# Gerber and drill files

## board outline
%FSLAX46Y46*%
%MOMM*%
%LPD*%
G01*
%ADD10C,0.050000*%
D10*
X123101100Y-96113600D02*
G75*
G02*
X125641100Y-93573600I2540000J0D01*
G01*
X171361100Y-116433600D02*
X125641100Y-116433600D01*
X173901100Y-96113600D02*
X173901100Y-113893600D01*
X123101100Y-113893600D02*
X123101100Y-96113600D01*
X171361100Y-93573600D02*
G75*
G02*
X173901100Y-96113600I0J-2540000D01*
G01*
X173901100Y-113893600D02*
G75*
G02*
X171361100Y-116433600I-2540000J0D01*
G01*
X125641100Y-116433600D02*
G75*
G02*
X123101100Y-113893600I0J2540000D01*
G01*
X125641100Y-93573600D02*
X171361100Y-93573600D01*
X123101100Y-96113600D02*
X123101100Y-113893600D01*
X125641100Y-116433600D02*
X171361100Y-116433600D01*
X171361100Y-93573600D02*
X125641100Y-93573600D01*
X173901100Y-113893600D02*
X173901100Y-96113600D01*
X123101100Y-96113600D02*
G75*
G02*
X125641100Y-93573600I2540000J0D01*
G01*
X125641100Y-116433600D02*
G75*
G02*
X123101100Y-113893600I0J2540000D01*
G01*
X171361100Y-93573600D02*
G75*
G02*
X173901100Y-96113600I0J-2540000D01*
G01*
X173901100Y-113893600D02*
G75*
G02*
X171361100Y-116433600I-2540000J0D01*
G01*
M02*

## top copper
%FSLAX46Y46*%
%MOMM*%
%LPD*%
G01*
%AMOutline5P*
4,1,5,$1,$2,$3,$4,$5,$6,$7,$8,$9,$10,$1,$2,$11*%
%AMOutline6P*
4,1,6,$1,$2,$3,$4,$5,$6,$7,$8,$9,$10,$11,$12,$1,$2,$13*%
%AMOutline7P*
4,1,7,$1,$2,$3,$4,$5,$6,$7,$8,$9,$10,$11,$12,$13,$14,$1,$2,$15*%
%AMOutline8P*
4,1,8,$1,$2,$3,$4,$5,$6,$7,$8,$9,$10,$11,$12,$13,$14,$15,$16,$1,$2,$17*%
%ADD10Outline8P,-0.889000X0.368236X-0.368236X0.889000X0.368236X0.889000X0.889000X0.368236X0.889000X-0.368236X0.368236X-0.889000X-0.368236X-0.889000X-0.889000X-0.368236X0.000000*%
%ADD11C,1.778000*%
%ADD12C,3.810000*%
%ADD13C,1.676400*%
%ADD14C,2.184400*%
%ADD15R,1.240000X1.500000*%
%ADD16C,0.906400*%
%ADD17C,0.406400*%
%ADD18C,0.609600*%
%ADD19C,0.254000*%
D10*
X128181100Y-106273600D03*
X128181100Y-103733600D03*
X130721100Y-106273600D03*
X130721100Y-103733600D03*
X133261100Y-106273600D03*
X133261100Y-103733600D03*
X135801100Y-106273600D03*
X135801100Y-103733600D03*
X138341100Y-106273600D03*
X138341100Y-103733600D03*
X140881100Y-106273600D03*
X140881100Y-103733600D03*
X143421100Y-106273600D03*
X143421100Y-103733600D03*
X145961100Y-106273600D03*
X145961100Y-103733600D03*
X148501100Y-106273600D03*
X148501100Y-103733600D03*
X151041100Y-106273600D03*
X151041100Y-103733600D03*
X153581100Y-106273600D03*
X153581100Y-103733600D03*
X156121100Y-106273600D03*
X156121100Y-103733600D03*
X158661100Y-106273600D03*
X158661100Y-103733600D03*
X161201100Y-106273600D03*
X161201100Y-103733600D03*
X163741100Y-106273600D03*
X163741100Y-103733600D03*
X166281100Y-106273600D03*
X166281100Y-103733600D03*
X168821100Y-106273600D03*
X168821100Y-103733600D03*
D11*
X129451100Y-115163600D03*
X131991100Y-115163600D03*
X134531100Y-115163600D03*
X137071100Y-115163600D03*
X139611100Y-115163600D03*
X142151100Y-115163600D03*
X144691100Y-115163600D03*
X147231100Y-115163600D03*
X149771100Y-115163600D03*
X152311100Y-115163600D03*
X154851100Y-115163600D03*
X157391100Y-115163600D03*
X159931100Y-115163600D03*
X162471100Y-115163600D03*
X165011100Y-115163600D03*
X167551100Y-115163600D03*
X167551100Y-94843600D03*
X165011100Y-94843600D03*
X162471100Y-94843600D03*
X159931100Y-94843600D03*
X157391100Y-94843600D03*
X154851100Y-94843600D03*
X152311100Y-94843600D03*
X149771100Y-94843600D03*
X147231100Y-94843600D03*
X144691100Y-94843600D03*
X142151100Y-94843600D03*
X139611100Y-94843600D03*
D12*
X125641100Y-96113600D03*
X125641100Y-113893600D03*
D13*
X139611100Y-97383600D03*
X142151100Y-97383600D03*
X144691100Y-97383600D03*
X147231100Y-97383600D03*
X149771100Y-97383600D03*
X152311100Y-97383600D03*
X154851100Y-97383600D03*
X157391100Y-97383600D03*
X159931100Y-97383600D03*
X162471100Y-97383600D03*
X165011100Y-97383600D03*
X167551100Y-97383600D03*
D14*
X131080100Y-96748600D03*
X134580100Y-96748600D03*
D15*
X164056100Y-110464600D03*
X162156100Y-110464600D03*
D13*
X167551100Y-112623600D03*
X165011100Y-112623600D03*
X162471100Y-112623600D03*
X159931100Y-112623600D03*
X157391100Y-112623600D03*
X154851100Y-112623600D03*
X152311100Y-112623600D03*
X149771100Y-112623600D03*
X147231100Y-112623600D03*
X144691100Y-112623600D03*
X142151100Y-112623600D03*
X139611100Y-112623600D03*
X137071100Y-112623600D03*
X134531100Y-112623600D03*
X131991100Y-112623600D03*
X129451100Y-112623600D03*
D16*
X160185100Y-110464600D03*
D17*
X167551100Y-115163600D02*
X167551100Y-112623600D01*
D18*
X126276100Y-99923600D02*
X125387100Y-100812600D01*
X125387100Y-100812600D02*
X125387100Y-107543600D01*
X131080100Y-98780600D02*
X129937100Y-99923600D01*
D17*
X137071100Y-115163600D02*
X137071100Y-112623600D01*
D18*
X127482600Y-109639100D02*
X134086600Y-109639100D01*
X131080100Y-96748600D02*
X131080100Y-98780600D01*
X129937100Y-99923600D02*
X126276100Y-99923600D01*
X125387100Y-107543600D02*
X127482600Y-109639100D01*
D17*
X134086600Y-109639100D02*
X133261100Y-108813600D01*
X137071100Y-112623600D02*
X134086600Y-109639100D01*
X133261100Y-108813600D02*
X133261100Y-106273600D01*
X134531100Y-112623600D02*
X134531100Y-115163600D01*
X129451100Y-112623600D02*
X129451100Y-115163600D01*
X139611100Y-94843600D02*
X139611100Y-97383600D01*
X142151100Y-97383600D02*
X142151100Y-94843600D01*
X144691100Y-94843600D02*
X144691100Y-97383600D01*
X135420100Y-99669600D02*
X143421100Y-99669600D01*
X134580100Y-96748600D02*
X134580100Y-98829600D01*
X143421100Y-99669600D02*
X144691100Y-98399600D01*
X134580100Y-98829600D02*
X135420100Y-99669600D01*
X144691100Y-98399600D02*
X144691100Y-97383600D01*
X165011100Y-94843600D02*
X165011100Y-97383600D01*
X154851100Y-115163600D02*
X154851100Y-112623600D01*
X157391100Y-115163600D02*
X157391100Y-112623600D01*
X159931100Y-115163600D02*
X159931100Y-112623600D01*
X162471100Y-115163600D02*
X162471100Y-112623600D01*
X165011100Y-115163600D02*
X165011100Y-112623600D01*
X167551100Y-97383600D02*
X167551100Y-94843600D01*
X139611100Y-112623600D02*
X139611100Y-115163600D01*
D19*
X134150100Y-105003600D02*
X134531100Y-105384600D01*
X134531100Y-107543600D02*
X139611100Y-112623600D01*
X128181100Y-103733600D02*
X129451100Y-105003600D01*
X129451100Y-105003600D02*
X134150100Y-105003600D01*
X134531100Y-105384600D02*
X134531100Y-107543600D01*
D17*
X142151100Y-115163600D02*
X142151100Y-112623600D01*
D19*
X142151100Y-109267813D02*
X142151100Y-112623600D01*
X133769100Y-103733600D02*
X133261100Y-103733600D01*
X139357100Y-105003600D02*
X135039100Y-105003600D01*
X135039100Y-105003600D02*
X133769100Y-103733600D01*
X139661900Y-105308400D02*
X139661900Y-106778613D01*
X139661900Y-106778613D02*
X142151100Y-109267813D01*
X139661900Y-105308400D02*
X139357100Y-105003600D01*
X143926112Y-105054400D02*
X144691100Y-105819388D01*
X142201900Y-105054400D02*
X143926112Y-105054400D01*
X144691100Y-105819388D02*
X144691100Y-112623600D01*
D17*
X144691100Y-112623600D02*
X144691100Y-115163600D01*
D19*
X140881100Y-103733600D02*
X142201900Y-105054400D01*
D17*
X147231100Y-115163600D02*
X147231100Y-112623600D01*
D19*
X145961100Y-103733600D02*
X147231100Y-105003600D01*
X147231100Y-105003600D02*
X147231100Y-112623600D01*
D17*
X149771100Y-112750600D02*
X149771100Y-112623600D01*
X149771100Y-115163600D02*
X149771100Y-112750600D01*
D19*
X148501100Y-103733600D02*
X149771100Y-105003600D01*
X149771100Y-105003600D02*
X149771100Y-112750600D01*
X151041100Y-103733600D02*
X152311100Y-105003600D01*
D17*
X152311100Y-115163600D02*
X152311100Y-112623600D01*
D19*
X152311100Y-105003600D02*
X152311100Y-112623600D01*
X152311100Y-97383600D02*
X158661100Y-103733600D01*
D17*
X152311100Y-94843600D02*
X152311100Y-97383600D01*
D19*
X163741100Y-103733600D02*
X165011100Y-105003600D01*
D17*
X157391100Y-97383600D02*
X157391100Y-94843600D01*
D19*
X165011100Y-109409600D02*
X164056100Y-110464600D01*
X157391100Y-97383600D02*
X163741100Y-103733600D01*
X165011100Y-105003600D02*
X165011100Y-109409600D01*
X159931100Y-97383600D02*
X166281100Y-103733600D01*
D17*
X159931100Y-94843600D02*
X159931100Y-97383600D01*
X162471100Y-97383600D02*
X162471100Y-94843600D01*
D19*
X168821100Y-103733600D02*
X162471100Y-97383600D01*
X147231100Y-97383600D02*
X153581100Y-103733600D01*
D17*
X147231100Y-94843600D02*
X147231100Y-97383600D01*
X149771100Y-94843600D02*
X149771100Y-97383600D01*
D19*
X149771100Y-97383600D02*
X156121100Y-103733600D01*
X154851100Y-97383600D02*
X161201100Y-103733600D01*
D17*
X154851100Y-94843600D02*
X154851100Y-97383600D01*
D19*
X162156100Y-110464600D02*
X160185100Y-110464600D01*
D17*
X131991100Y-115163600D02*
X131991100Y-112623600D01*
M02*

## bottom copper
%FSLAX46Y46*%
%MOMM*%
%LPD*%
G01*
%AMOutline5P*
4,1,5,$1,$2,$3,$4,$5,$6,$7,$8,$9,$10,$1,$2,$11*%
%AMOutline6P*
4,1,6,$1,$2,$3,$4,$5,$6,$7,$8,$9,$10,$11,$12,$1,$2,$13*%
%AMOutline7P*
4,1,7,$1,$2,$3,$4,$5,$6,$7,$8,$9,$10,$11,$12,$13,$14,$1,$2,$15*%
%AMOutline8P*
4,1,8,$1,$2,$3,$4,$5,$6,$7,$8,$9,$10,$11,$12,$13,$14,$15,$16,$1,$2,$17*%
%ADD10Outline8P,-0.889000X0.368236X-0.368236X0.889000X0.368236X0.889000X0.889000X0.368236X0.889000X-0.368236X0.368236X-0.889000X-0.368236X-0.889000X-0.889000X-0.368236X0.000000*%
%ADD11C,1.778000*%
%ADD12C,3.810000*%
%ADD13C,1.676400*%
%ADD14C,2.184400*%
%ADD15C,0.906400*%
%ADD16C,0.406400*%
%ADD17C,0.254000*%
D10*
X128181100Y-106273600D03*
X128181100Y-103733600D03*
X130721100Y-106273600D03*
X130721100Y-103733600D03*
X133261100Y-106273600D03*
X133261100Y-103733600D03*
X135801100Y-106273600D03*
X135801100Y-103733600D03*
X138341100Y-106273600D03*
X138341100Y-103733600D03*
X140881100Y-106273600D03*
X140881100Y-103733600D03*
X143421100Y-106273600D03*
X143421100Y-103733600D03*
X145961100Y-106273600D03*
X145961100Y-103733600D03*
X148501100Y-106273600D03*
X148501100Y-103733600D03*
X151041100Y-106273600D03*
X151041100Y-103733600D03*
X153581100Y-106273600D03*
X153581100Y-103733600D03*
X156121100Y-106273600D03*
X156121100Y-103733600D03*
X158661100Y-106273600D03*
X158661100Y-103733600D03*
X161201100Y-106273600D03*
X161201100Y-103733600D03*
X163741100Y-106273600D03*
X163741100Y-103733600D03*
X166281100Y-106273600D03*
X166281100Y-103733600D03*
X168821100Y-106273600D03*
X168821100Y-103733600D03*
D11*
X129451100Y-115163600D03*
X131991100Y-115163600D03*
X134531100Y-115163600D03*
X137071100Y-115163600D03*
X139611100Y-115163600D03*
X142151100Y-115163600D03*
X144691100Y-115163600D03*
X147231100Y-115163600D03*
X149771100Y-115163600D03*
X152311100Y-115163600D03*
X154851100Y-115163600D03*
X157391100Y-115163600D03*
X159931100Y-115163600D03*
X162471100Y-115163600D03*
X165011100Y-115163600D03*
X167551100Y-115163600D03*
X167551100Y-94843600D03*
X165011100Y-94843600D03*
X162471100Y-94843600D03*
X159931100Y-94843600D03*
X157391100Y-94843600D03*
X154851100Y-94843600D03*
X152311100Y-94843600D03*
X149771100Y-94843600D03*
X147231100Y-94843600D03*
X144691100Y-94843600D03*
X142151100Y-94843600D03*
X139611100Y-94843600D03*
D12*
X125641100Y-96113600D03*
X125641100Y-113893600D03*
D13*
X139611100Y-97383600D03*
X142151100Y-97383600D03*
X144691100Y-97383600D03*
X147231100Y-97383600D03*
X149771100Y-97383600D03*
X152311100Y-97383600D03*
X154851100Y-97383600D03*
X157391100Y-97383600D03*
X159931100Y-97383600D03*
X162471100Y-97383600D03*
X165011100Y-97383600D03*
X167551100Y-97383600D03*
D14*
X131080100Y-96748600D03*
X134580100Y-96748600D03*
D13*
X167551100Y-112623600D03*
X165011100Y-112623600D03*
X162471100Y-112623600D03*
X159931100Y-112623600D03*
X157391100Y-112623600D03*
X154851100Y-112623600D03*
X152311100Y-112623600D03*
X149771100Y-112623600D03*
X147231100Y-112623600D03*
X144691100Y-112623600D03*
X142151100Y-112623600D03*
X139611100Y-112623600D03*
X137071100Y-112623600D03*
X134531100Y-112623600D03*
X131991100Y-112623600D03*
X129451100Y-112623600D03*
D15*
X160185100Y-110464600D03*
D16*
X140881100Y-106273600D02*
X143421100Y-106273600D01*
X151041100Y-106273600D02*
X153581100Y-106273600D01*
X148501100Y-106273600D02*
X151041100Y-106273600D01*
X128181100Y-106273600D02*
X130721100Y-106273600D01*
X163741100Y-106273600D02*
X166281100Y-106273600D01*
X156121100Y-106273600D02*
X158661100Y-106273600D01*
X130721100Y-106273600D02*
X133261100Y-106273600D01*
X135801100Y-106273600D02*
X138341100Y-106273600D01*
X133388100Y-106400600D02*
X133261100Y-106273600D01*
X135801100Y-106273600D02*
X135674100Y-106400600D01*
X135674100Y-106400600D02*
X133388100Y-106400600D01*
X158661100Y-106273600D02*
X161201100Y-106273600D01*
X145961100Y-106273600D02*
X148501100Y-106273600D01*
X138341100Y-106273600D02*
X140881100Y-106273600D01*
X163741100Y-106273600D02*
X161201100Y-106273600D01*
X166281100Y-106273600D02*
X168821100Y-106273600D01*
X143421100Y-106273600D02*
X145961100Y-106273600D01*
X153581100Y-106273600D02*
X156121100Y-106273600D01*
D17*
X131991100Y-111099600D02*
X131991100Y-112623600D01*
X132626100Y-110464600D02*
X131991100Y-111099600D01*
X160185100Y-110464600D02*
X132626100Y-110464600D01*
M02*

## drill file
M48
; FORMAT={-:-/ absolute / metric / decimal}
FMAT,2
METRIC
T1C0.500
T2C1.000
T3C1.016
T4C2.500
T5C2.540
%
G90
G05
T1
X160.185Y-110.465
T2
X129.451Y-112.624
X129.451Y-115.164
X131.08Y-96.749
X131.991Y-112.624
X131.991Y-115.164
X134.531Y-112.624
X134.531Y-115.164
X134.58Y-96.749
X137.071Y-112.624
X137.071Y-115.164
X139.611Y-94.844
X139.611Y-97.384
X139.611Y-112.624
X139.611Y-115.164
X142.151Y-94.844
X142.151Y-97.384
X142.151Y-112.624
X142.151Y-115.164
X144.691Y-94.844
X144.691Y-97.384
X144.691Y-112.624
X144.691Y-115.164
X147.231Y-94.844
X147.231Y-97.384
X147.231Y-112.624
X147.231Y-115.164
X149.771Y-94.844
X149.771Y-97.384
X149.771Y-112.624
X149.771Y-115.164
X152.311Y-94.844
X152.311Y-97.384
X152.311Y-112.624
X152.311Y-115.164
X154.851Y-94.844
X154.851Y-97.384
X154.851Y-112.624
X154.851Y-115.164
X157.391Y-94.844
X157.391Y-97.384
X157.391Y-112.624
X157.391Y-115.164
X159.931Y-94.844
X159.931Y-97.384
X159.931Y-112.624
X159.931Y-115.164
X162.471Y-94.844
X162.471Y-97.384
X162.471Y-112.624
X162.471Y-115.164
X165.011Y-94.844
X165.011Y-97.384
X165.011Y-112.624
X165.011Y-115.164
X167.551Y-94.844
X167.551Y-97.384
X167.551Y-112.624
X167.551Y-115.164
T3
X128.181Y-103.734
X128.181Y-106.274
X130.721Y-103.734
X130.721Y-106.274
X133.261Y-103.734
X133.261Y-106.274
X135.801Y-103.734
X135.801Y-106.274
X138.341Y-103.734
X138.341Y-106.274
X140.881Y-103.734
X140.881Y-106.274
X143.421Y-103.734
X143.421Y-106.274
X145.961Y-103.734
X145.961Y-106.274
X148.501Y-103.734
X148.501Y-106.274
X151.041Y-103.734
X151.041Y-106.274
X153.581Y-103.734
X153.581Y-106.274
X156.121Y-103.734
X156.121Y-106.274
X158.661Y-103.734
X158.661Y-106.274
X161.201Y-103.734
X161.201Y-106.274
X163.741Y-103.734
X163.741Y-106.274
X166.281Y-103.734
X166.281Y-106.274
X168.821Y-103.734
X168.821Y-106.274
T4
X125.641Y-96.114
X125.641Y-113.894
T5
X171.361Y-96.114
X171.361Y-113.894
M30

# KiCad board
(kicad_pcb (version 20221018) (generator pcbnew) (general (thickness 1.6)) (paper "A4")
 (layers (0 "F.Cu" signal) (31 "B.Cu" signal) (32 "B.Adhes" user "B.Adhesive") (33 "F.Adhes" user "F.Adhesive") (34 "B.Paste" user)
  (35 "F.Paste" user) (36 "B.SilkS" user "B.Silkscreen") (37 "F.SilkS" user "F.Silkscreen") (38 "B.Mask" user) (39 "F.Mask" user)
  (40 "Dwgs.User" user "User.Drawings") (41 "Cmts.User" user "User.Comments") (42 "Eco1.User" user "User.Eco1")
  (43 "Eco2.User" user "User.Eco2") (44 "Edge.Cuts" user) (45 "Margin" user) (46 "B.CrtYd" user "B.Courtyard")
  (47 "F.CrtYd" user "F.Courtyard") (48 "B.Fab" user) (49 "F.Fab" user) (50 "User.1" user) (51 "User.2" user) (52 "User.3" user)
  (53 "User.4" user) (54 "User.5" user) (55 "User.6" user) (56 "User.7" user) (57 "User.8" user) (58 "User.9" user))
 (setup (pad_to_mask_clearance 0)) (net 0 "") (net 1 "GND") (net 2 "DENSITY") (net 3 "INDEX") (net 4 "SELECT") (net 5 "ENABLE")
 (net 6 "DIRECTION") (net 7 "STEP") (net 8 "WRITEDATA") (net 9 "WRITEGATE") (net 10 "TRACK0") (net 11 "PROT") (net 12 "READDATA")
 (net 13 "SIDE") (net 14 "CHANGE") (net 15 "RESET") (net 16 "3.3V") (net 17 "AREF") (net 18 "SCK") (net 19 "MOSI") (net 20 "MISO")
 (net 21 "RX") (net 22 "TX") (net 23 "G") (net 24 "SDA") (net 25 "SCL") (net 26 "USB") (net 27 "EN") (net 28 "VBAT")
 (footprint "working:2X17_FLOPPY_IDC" (layer "F.Cu") (at 148.5011 105.0036 90)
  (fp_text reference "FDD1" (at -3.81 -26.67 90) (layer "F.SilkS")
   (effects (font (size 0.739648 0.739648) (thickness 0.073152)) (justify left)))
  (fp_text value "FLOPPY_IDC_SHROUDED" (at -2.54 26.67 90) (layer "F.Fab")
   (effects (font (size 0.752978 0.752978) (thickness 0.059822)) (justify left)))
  (pad "1" thru_hole roundrect (at -1.27 -20.32) (size 1.778 1.778) (drill 1.016) (layers "*.Cu" "*.Mask") (roundrect_rratio 0.25)
   (chamfer_ratio 0.2928932188) (chamfer top_left top_right bottom_left bottom_right) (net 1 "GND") (solder_mask_margin 0.0508)
   (thermal_bridge_angle 45))
  (pad "2" thru_hole roundrect (at 1.27 -20.32) (size 1.778 1.778) (drill 1.016) (layers "*.Cu" "*.Mask") (roundrect_rratio 0.25)
   (chamfer_ratio 0.2928932188) (chamfer top_left top_right bottom_left bottom_right) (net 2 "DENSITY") (solder_mask_margin 0.0508)
   (thermal_bridge_angle 45))
  (pad "3" thru_hole roundrect (at -1.27 -17.78) (size 1.778 1.778) (drill 1.016) (layers "*.Cu" "*.Mask") (roundrect_rratio 0.25)
   (chamfer_ratio 0.2928932188) (chamfer top_left top_right bottom_left bottom_right) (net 1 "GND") (solder_mask_margin 0.0508)
   (thermal_bridge_angle 45))
  (pad "4" thru_hole roundrect (at 1.27 -17.78) (size 1.778 1.778) (drill 1.016) (layers "*.Cu" "*.Mask") (roundrect_rratio 0.25)
   (chamfer_ratio 0.2928932188) (chamfer top_left top_right bottom_left bottom_right) (solder_mask_margin 0.0508) (thermal_bridge_angle 45))
  (pad "5" thru_hole roundrect (at -1.27 -15.24) (size 1.778 1.778) (drill 1.016) (layers "*.Cu" "*.Mask") (roundrect_rratio 0.25)
   (chamfer_ratio 0.2928932188) (chamfer top_left top_right bottom_left bottom_right) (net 1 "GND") (solder_mask_margin 0.0508)
   (thermal_bridge_angle 45))
  (pad "6" thru_hole roundrect (at 1.27 -15.24) (size 1.778 1.778) (drill 1.016) (layers "*.Cu" "*.Mask") (roundrect_rratio 0.25)
   (chamfer_ratio 0.2928932188) (chamfer top_left top_right bottom_left bottom_right) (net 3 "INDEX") (solder_mask_margin 0.0508)
   (thermal_bridge_angle 45))
  (pad "7" thru_hole roundrect (at -1.27 -12.7) (size 1.778 1.778) (drill 1.016) (layers "*.Cu" "*.Mask") (roundrect_rratio 0.25)
   (chamfer_ratio 0.2928932188) (chamfer top_left top_right bottom_left bottom_right) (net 1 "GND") (solder_mask_margin 0.0508)
   (thermal_bridge_angle 45))
  (pad "8" thru_hole roundrect (at 1.27 -12.7) (size 1.778 1.778) (drill 1.016) (layers "*.Cu" "*.Mask") (roundrect_rratio 0.25)
   (chamfer_ratio 0.2928932188) (chamfer top_left top_right bottom_left bottom_right) (solder_mask_margin 0.0508) (thermal_bridge_angle 45))
  (pad "9" thru_hole roundrect (at -1.27 -10.16) (size 1.778 1.778) (drill 1.016) (layers "*.Cu" "*.Mask") (roundrect_rratio 0.25)
   (chamfer_ratio 0.2928932188) (chamfer top_left top_right bottom_left bottom_right) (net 1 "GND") (solder_mask_margin 0.0508)
   (thermal_bridge_angle 45))
  (pad "10" thru_hole roundrect (at 1.27 -10.16) (size 1.778 1.778) (drill 1.016) (layers "*.Cu" "*.Mask") (roundrect_rratio 0.25)
   (chamfer_ratio 0.2928932188) (chamfer top_left top_right bottom_left bottom_right) (solder_mask_margin 0.0508) (thermal_bridge_angle 45))
  (pad "11" thru_hole roundrect (at -1.27 -7.62) (size 1.778 1.778) (drill 1.016) (layers "*.Cu" "*.Mask") (roundrect_rratio 0.25)
   (chamfer_ratio 0.2928932188) (chamfer top_left top_right bottom_left bottom_right) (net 1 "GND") (solder_mask_margin 0.0508)
   (thermal_bridge_angle 45))
  (pad "12" thru_hole roundrect (at 1.27 -7.62) (size 1.778 1.778) (drill 1.016) (layers "*.Cu" "*.Mask") (roundrect_rratio 0.25)
   (chamfer_ratio 0.2928932188) (chamfer top_left top_right bottom_left bottom_right) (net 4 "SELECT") (solder_mask_margin 0.0508)
   (thermal_bridge_angle 45))
  (pad "13" thru_hole roundrect (at -1.27 -5.08) (size 1.778 1.778) (drill 1.016) (layers "*.Cu" "*.Mask") (roundrect_rratio 0.25)
   (chamfer_ratio 0.2928932188) (chamfer top_left top_right bottom_left bottom_right) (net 1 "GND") (solder_mask_margin 0.0508)
   (thermal_bridge_angle 45))
  (pad "14" thru_hole roundrect (at 1.27 -5.08) (size 1.778 1.778) (drill 1.016) (layers "*.Cu" "*.Mask") (roundrect_rratio 0.25)
   (chamfer_ratio 0.2928932188) (chamfer top_left top_right bottom_left bottom_right) (solder_mask_margin 0.0508) (thermal_bridge_angle 45))
  (pad "15" thru_hole roundrect (at -1.27 -2.54) (size 1.778 1.778) (drill 1.016) (layers "*.Cu" "*.Mask") (roundrect_rratio 0.25)
   (chamfer_ratio 0.2928932188) (chamfer top_left top_right bottom_left bottom_right) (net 1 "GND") (solder_mask_margin 0.0508)
   (thermal_bridge_angle 45))
  (pad "16" thru_hole roundrect (at 1.27 -2.54) (size 1.778 1.778) (drill 1.016) (layers "*.Cu" "*.Mask") (roundrect_rratio 0.25)
   (chamfer_ratio 0.2928932188) (chamfer top_left top_right bottom_left bottom_right) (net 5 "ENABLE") (solder_mask_margin 0.0508)
   (thermal_bridge_angle 45))
  (pad "17" thru_hole roundrect (at -1.27 0) (size 1.778 1.778) (drill 1.016) (layers "*.Cu" "*.Mask") (roundrect_rratio 0.25)
   (chamfer_ratio 0.2928932188) (chamfer top_left top_right bottom_left bottom_right) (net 1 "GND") (solder_mask_margin 0.0508)
   (thermal_bridge_angle 45))
  (pad "18" thru_hole roundrect (at 1.27 0) (size 1.778 1.778) (drill 1.016) (layers "*.Cu" "*.Mask") (roundrect_rratio 0.25)
   (chamfer_ratio 0.2928932188) (chamfer top_left top_right bottom_left bottom_right) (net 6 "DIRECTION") (solder_mask_margin 0.0508)
   (thermal_bridge_angle 45))
  (pad "19" thru_hole roundrect (at -1.27 2.54) (size 1.778 1.778) (drill 1.016) (layers "*.Cu" "*.Mask") (roundrect_rratio 0.25)
   (chamfer_ratio 0.2928932188) (chamfer top_left top_right bottom_left bottom_right) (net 1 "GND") (solder_mask_margin 0.0508)
   (thermal_bridge_angle 45))
  (pad "20" thru_hole roundrect (at 1.27 2.54) (size 1.778 1.778) (drill 1.016) (layers "*.Cu" "*.Mask") (roundrect_rratio 0.25)
   (chamfer_ratio 0.2928932188) (chamfer top_left top_right bottom_left bottom_right) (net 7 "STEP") (solder_mask_margin 0.0508)
   (thermal_bridge_angle 45))
  (pad "21" thru_hole roundrect (at -1.27 5.08) (size 1.778 1.778) (drill 1.016) (layers "*.Cu" "*.Mask") (roundrect_rratio 0.25)
   (chamfer_ratio 0.2928932188) (chamfer top_left top_right bottom_left bottom_right) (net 1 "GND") (solder_mask_margin 0.0508)
   (thermal_bridge_angle 45))
  (pad "22" thru_hole roundrect (at 1.27 5.08) (size 1.778 1.778) (drill 1.016) (layers "*.Cu" "*.Mask") (roundrect_rratio 0.25)
   (chamfer_ratio 0.2928932188) (chamfer top_left top_right bottom_left bottom_right) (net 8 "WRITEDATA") (solder_mask_margin 0.0508)
   (thermal_bridge_angle 45))
  (pad "23" thru_hole roundrect (at -1.27 7.62) (size 1.778 1.778) (drill 1.016) (layers "*.Cu" "*.Mask") (roundrect_rratio 0.25)
   (chamfer_ratio 0.2928932188) (chamfer top_left top_right bottom_left bottom_right) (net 1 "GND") (solder_mask_margin 0.0508)
   (thermal_bridge_angle 45))
  (pad "24" thru_hole roundrect (at 1.27 7.62) (size 1.778 1.778) (drill 1.016) (layers "*.Cu" "*.Mask") (roundrect_rratio 0.25)
   (chamfer_ratio 0.2928932188) (chamfer top_left top_right bottom_left bottom_right) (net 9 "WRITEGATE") (solder_mask_margin 0.0508)
   (thermal_bridge_angle 45))
  (pad "25" thru_hole roundrect (at -1.27 10.16) (size 1.778 1.778) (drill 1.016) (layers "*.Cu" "*.Mask") (roundrect_rratio 0.25)
   (chamfer_ratio 0.2928932188) (chamfer top_left top_right bottom_left bottom_right) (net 1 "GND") (solder_mask_margin 0.0508)
   (thermal_bridge_angle 45))
  (pad "26" thru_hole roundrect (at 1.27 10.16) (size 1.778 1.778) (drill 1.016) (layers "*.Cu" "*.Mask") (roundrect_rratio 0.25)
   (chamfer_ratio 0.2928932188) (chamfer top_left top_right bottom_left bottom_right) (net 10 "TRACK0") (solder_mask_margin 0.0508)
   (thermal_bridge_angle 45))
  (pad "27" thru_hole roundrect (at -1.27 12.7) (size 1.778 1.778) (drill 1.016) (layers "*.Cu" "*.Mask") (roundrect_rratio 0.25)
   (chamfer_ratio 0.2928932188) (chamfer top_left top_right bottom_left bottom_right) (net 1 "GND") (solder_mask_margin 0.0508)
   (thermal_bridge_angle 45))
  (pad "28" thru_hole roundrect (at 1.27 12.7) (size 1.778 1.778) (drill 1.016) (layers "*.Cu" "*.Mask") (roundrect_rratio 0.25)
   (chamfer_ratio 0.2928932188) (chamfer top_left top_right bottom_left bottom_right) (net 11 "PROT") (solder_mask_margin 0.0508)
   (thermal_bridge_angle 45))
  (pad "29" thru_hole roundrect (at -1.27 15.24) (size 1.778 1.778) (drill 1.016) (layers "*.Cu" "*.Mask") (roundrect_rratio 0.25)
   (chamfer_ratio 0.2928932188) (chamfer top_left top_right bottom_left bottom_right) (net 1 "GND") (solder_mask_margin 0.0508)
   (thermal_bridge_angle 45))
  (pad "30" thru_hole roundrect (at 1.27 15.24) (size 1.778 1.778) (drill 1.016) (layers "*.Cu" "*.Mask") (roundrect_rratio 0.25)
   (chamfer_ratio 0.2928932188) (chamfer top_left top_right bottom_left bottom_right) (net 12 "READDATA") (solder_mask_margin 0.0508)
   (thermal_bridge_angle 45))
  (pad "31" thru_hole roundrect (at -1.27 17.78) (size 1.778 1.778) (drill 1.016) (layers "*.Cu" "*.Mask") (roundrect_rratio 0.25)
   (chamfer_ratio 0.2928932188) (chamfer top_left top_right bottom_left bottom_right) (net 1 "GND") (solder_mask_margin 0.0508)
   (thermal_bridge_angle 45))
  (pad "32" thru_hole roundrect (at 1.27 17.78) (size 1.778 1.778) (drill 1.016) (layers "*.Cu" "*.Mask") (roundrect_rratio 0.25)
   (chamfer_ratio 0.2928932188) (chamfer top_left top_right bottom_left bottom_right) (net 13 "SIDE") (solder_mask_margin 0.0508)
   (thermal_bridge_angle 45))
  (pad "33" thru_hole roundrect (at -1.27 20.32) (size 1.778 1.778) (drill 1.016) (layers "*.Cu" "*.Mask") (roundrect_rratio 0.25)
   (chamfer_ratio 0.2928932188) (chamfer top_left top_right bottom_left bottom_right) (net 1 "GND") (solder_mask_margin 0.0508)
   (thermal_bridge_angle 45))
  (pad "34" thru_hole roundrect (at 1.27 20.32) (size 1.778 1.778) (drill 1.016) (layers "*.Cu" "*.Mask") (roundrect_rratio 0.25)
   (chamfer_ratio 0.2928932188) (chamfer top_left top_right bottom_left bottom_right) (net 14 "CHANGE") (solder_mask_margin 0.0508)
   (thermal_bridge_angle 45)))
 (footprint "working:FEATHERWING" (layer "F.Cu") (at 123.1011 116.4336)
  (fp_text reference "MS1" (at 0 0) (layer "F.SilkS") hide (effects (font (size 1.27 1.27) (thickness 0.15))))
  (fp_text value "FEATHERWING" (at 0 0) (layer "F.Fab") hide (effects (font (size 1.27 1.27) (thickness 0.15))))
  (fp_line (start 0 -20.32) (end 0 -2.54) (stroke (width 0.05) (type solid)) (layer "Edge.Cuts"))
  (fp_line (start 2.54 0) (end 48.26 0) (stroke (width 0.05) (type solid)) (layer "Edge.Cuts"))
  (fp_line (start 48.26 -22.86) (end 2.54 -22.86) (stroke (width 0.05) (type solid)) (layer "Edge.Cuts"))
  (fp_line (start 50.8 -2.54) (end 50.8 -20.32) (stroke (width 0.05) (type solid)) (layer "Edge.Cuts"))
  (fp_arc (start 0 -20.32) (mid 0.743949 -22.116051) (end 2.54 -22.86) (stroke (width 0.05) (type solid)) (layer "Edge.Cuts"))
  (fp_arc (start 2.54 0) (mid 0.743949 -0.743949) (end 0 -2.54) (stroke (width 0.05) (type solid)) (layer "Edge.Cuts"))
  (fp_arc (start 48.26 -22.86) (mid 50.056051 -22.116051) (end 50.8 -20.32) (stroke (width 0.05) (type solid)) (layer "Edge.Cuts"))
  (fp_arc (start 50.8 -2.54) (mid 50.056051 -0.743949) (end 48.26 0) (stroke (width 0.05) (type solid)) (layer "Edge.Cuts"))
  (pad "" np_thru_hole circle (at 48.26 -20.32) (size 2.54 2.54) (drill 2.54) (layers "*.Cu" "*.Mask"))
  (pad "" np_thru_hole circle (at 48.26 -2.54) (size 2.54 2.54) (drill 2.54) (layers "*.Cu" "*.Mask"))
  (pad "1" thru_hole circle (at 6.35 -1.27) (size 1.778 1.778) (drill 1) (layers "*.Cu" "*.Mask") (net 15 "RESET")
   (solder_mask_margin 0.0508))
  (pad "2" thru_hole circle (at 8.89 -1.27) (size 1.778 1.778) (drill 1) (layers "*.Cu" "*.Mask") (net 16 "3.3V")
   (solder_mask_margin 0.0508))
  (pad "3" thru_hole circle (at 11.43 -1.27) (size 1.778 1.778) (drill 1) (layers "*.Cu" "*.Mask") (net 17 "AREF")
   (solder_mask_margin 0.0508))
  (pad "4" thru_hole circle (at 13.97 -1.27) (size 1.778 1.778) (drill 1) (layers "*.Cu" "*.Mask") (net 1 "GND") (solder_mask_margin 0.0508))
  (pad "5" thru_hole circle (at 16.51 -1.27) (size 1.778 1.778) (drill 1) (layers "*.Cu" "*.Mask") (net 2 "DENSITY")
   (solder_mask_margin 0.0508))
  (pad "6" thru_hole circle (at 19.05 -1.27) (size 1.778 1.778) (drill 1) (layers "*.Cu" "*.Mask") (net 3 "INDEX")
   (solder_mask_margin 0.0508))
  (pad "7" thru_hole circle (at 21.59 -1.27) (size 1.778 1.778) (drill 1) (layers "*.Cu" "*.Mask") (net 4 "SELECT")
   (solder_mask_margin 0.0508))
  (pad "8" thru_hole circle (at 24.13 -1.27) (size 1.778 1.778) (drill 1) (layers "*.Cu" "*.Mask") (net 5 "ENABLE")
   (solder_mask_margin 0.0508))
  (pad "9" thru_hole circle (at 26.67 -1.27) (size 1.778 1.778) (drill 1) (layers "*.Cu" "*.Mask") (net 6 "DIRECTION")
   (solder_mask_margin 0.0508))
  (pad "10" thru_hole circle (at 29.21 -1.27) (size 1.778 1.778) (drill 1) (layers "*.Cu" "*.Mask") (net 7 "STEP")
   (solder_mask_margin 0.0508))
  (pad "11" thru_hole circle (at 31.75 -1.27) (size 1.778 1.778) (drill 1) (layers "*.Cu" "*.Mask") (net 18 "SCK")
   (solder_mask_margin 0.0508))
  (pad "12" thru_hole circle (at 34.29 -1.27) (size 1.778 1.778) (drill 1) (layers "*.Cu" "*.Mask") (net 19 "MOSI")
   (solder_mask_margin 0.0508))
  (pad "13" thru_hole circle (at 36.83 -1.27) (size 1.778 1.778) (drill 1) (layers "*.Cu" "*.Mask") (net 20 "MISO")
   (solder_mask_margin 0.0508))
  (pad "14" thru_hole circle (at 39.37 -1.27) (size 1.778 1.778) (drill 1) (layers "*.Cu" "*.Mask") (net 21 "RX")
   (solder_mask_margin 0.0508))
  (pad "15" thru_hole circle (at 41.91 -1.27) (size 1.778 1.778) (drill 1) (layers "*.Cu" "*.Mask") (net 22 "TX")
   (solder_mask_margin 0.0508))
  (pad "16" thru_hole circle (at 44.45 -1.27) (size 1.778 1.778) (drill 1) (layers "*.Cu" "*.Mask") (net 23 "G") (solder_mask_margin 0.0508))
  (pad "17" thru_hole circle (at 44.45 -21.59) (size 1.778 1.778) (drill 1) (layers "*.Cu" "*.Mask") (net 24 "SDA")
   (solder_mask_margin 0.0508))
  (pad "18" thru_hole circle (at 41.91 -21.59) (size 1.778 1.778) (drill 1) (layers "*.Cu" "*.Mask") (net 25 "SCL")
   (solder_mask_margin 0.0508))
  (pad "19" thru_hole circle (at 39.37 -21.59) (size 1.778 1.778) (drill 1) (layers "*.Cu" "*.Mask") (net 14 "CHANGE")
   (solder_mask_margin 0.0508))
  (pad "20" thru_hole circle (at 36.83 -21.59) (size 1.778 1.778) (drill 1) (layers "*.Cu" "*.Mask") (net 13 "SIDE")
   (solder_mask_margin 0.0508))
  (pad "21" thru_hole circle (at 34.29 -21.59) (size 1.778 1.778) (drill 1) (layers "*.Cu" "*.Mask") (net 12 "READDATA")
   (solder_mask_margin 0.0508))
  (pad "22" thru_hole circle (at 31.75 -21.59) (size 1.778 1.778) (drill 1) (layers "*.Cu" "*.Mask") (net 11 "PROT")
   (solder_mask_margin 0.0508))
  (pad "23" thru_hole circle (at 29.21 -21.59) (size 1.778 1.778) (drill 1) (layers "*.Cu" "*.Mask") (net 10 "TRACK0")
   (solder_mask_margin 0.0508))
  (pad "24" thru_hole circle (at 26.67 -21.59) (size 1.778 1.778) (drill 1) (layers "*.Cu" "*.Mask") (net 9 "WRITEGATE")
   (solder_mask_margin 0.0508))
  (pad "25" thru_hole circle (at 24.13 -21.59) (size 1.778 1.778) (drill 1) (layers "*.Cu" "*.Mask") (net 8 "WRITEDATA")
   (solder_mask_margin 0.0508))
  (pad "26" thru_hole circle (at 21.59 -21.59) (size 1.778 1.778) (drill 1) (layers "*.Cu" "*.Mask") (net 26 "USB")
   (solder_mask_margin 0.0508))
  (pad "27" thru_hole circle (at 19.05 -21.59) (size 1.778 1.778) (drill 1) (layers "*.Cu" "*.Mask") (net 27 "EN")
   (solder_mask_margin 0.0508))
  (pad "28" thru_hole circle (at 16.51 -21.59) (size 1.778 1.778) (drill 1) (layers "*.Cu" "*.Mask") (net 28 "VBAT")
   (solder_mask_margin 0.0508))
  (pad "P$1" thru_hole circle (at 2.54 -20.32) (size 3.81 3.81) (drill 2.5) (layers "*.Cu" "*.Mask") (solder_mask_margin 0.0508))
  (pad "P$2" thru_hole circle (at 2.54 -2.54) (size 3.81 3.81) (drill 2.5) (layers "*.Cu" "*.Mask") (solder_mask_margin 0.0508)))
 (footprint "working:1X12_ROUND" (layer "F.Cu") (at 153.5811 97.3836)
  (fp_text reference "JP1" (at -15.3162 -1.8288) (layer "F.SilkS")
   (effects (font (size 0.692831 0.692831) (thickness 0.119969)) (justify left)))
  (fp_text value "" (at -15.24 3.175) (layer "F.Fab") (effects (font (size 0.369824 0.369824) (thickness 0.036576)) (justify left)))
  (pad "1" thru_hole circle (at -13.97 0 90) (size 1.6764 1.6764) (drill 1) (layers "*.Cu" "*.Mask") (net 28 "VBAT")
   (solder_mask_margin 0.0508))
  (pad "2" thru_hole circle (at -11.43 0 90) (size 1.6764 1.6764) (drill 1) (layers "*.Cu" "*.Mask") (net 27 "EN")
   (solder_mask_margin 0.0508))
  (pad "3" thru_hole circle (at -8.89 0 90) (size 1.6764 1.6764) (drill 1) (layers "*.Cu" "*.Mask") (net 26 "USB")
   (solder_mask_margin 0.0508))
  (pad "4" thru_hole circle (at -6.35 0 90) (size 1.6764 1.6764) (drill 1) (layers "*.Cu" "*.Mask") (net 8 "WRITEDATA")
   (solder_mask_margin 0.0508))
  (pad "5" thru_hole circle (at -3.81 0 90) (size 1.6764 1.6764) (drill 1) (layers "*.Cu" "*.Mask") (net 9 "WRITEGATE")
   (solder_mask_margin 0.0508))
  (pad "6" thru_hole circle (at -1.27 0 90) (size 1.6764 1.6764) (drill 1) (layers "*.Cu" "*.Mask") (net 10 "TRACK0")
   (solder_mask_margin 0.0508))
  (pad "7" thru_hole circle (at 1.27 0 90) (size 1.6764 1.6764) (drill 1) (layers "*.Cu" "*.Mask") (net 11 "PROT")
   (solder_mask_margin 0.0508))
  (pad "8" thru_hole circle (at 3.81 0 90) (size 1.6764 1.6764) (drill 1) (layers "*.Cu" "*.Mask") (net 12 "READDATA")
   (solder_mask_margin 0.0508))
  (pad "9" thru_hole circle (at 6.35 0 90) (size 1.6764 1.6764) (drill 1) (layers "*.Cu" "*.Mask") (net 13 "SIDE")
   (solder_mask_margin 0.0508))
  (pad "10" thru_hole circle (at 8.89 0 90) (size 1.6764 1.6764) (drill 1) (layers "*.Cu" "*.Mask") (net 14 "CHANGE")
   (solder_mask_margin 0.0508))
  (pad "11" thru_hole circle (at 11.43 0 90) (size 1.6764 1.6764) (drill 1) (layers "*.Cu" "*.Mask") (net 25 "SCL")
   (solder_mask_margin 0.0508))
  (pad "12" thru_hole circle (at 13.97 0 90) (size 1.6764 1.6764) (drill 1) (layers "*.Cu" "*.Mask") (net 24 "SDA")
   (solder_mask_margin 0.0508)))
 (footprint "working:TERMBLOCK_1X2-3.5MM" (layer "F.Cu") (at 132.8801 96.7486 180)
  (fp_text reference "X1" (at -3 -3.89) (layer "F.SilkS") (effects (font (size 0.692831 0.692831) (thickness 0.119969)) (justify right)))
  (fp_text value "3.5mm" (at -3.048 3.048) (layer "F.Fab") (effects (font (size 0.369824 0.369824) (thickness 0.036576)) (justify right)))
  (pad "1" thru_hole circle (at 1.8 0 180) (size 2.1844 2.1844) (drill 1) (layers "*.Cu" "*.Mask") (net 1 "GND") (solder_mask_margin 0.0508))
  (pad "2" thru_hole circle (at -1.7 0 180) (size 2.1844 2.1844) (drill 1) (layers "*.Cu" "*.Mask") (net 26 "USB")
   (solder_mask_margin 0.0508)))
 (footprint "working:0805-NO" (layer "F.Cu") (at 163.1061 110.4646 180)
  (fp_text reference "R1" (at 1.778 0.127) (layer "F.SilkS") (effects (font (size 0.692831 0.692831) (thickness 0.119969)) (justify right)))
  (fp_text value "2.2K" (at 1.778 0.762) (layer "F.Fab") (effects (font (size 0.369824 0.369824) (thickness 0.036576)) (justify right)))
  (pad "1" smd rect (at -0.95 0 180) (size 1.24 1.5) (layers "F.Cu" "F.Paste" "F.Mask") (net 12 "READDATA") (solder_mask_margin 0.0508)
   (thermal_bridge_angle 45))
  (pad "2" smd rect (at 0.95 0 180) (size 1.24 1.5) (layers "F.Cu" "F.Paste" "F.Mask") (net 16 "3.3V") (solder_mask_margin 0.0508)
   (thermal_bridge_angle 45)))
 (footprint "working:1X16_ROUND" (layer "F.Cu") (at 148.5011 112.6236 180)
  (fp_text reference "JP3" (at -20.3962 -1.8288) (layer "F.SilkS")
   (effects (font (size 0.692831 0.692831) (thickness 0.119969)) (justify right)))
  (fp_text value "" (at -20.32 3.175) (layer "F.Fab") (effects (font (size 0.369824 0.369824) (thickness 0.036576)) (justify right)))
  (pad "1" thru_hole circle (at -19.05 0 270) (size 1.6764 1.6764) (drill 1) (layers "*.Cu" "*.Mask") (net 23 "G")
   (solder_mask_margin 0.0508))
  (pad "2" thru_hole circle (at -16.51 0 270) (size 1.6764 1.6764) (drill 1) (layers "*.Cu" "*.Mask") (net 22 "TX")
   (solder_mask_margin 0.0508))
  (pad "3" thru_hole circle (at -13.97 0 270) (size 1.6764 1.6764) (drill 1) (layers "*.Cu" "*.Mask") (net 21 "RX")
   (solder_mask_margin 0.0508))
  (pad "4" thru_hole circle (at -11.43 0 270) (size 1.6764 1.6764) (drill 1) (layers "*.Cu" "*.Mask") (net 20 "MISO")
   (solder_mask_margin 0.0508))
  (pad "5" thru_hole circle (at -8.89 0 270) (size 1.6764 1.6764) (drill 1) (layers "*.Cu" "*.Mask") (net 19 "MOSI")
   (solder_mask_margin 0.0508))
  (pad "6" thru_hole circle (at -6.35 0 270) (size 1.6764 1.6764) (drill 1) (layers "*.Cu" "*.Mask") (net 18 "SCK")
   (solder_mask_margin 0.0508))
  (pad "7" thru_hole circle (at -3.81 0 270) (size 1.6764 1.6764) (drill 1) (layers "*.Cu" "*.Mask") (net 7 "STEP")
   (solder_mask_margin 0.0508))
  (pad "8" thru_hole circle (at -1.27 0 270) (size 1.6764 1.6764) (drill 1) (layers "*.Cu" "*.Mask") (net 6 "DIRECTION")
   (solder_mask_margin 0.0508))
  (pad "9" thru_hole circle (at 1.27 0 270) (size 1.6764 1.6764) (drill 1) (layers "*.Cu" "*.Mask") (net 5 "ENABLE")
   (solder_mask_margin 0.0508))
  (pad "10" thru_hole circle (at 3.81 0 270) (size 1.6764 1.6764) (drill 1) (layers "*.Cu" "*.Mask") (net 4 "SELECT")
   (solder_mask_margin 0.0508))
  (pad "11" thru_hole circle (at 6.35 0 270) (size 1.6764 1.6764) (drill 1) (layers "*.Cu" "*.Mask") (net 3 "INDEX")
   (solder_mask_margin 0.0508))
  (pad "12" thru_hole circle (at 8.89 0 270) (size 1.6764 1.6764) (drill 1) (layers "*.Cu" "*.Mask") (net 2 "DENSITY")
   (solder_mask_margin 0.0508))
  (pad "13" thru_hole circle (at 11.43 0 270) (size 1.6764 1.6764) (drill 1) (layers "*.Cu" "*.Mask") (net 1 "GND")
   (solder_mask_margin 0.0508))
  (pad "14" thru_hole circle (at 13.97 0 270) (size 1.6764 1.6764) (drill 1) (layers "*.Cu" "*.Mask") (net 17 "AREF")
   (solder_mask_margin 0.0508))
  (pad "15" thru_hole circle (at 16.51 0 270) (size 1.6764 1.6764) (drill 1) (layers "*.Cu" "*.Mask") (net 16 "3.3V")
   (solder_mask_margin 0.0508))
  (pad "16" thru_hole circle (at 19.05 0 270) (size 1.6764 1.6764) (drill 1) (layers "*.Cu" "*.Mask") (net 15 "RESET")
   (solder_mask_margin 0.0508)))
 (gr_arc (start 123.1011 96.1136) (mid 123.845049 94.317549) (end 125.6411 93.5736) (stroke (width 0.05) (type solid)) (layer "Edge.Cuts"))
 (gr_line (start 171.3611 116.4336) (end 125.6411 116.4336) (stroke (width 0.05) (type solid)) (layer "Edge.Cuts"))
 (gr_line (start 173.9011 96.1136) (end 173.9011 113.8936) (stroke (width 0.05) (type solid)) (layer "Edge.Cuts"))
 (gr_line (start 123.1011 113.8936) (end 123.1011 96.1136) (stroke (width 0.05) (type solid)) (layer "Edge.Cuts"))
 (gr_arc (start 171.3611 93.5736) (mid 173.157151 94.317549) (end 173.9011 96.1136) (stroke (width 0.05) (type solid)) (layer "Edge.Cuts"))
 (gr_arc (start 173.9011 113.8936) (mid 173.157151 115.689651) (end 171.3611 116.4336) (stroke (width 0.05) (type solid))
  (layer "Edge.Cuts"))
 (gr_arc (start 125.6411 116.4336) (mid 123.845049 115.689651) (end 123.1011 113.8936) (stroke (width 0.05) (type solid))
  (layer "Edge.Cuts"))
 (gr_line (start 125.6411 93.5736) (end 171.3611 93.5736) (stroke (width 0.05) (type solid)) (layer "Edge.Cuts"))
 (segment (start 167.5511 115.1636) (end 167.5511 112.6236) (width 0.4064) (layer "F.Cu") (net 23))
 (segment (start 126.2761 99.9236) (end 125.3871 100.8126) (width 0.6096) (layer "F.Cu") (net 1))
 (segment (start 125.3871 100.8126) (end 125.3871 107.5436) (width 0.6096) (layer "F.Cu") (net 1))
 (segment (start 131.0801 98.7806) (end 129.9371 99.9236) (width 0.6096) (layer "F.Cu") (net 1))
 (segment (start 137.0711 115.1636) (end 137.0711 112.6236) (width 0.4064) (layer "F.Cu") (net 1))
 (segment (start 127.4826 109.6391) (end 134.0866 109.6391) (width 0.6096) (layer "F.Cu") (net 1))
 (segment (start 131.0801 96.7486) (end 131.0801 98.7806) (width 0.6096) (layer "F.Cu") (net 1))
 (segment (start 129.9371 99.9236) (end 126.2761 99.9236) (width 0.6096) (layer "F.Cu") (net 1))
 (segment (start 125.3871 107.5436) (end 127.4826 109.6391) (width 0.6096) (layer "F.Cu") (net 1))
 (segment (start 134.0866 109.6391) (end 133.2611 108.8136) (width 0.4064) (layer "F.Cu") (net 1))
 (segment (start 137.0711 112.6236) (end 134.0866 109.6391) (width 0.4064) (layer "F.Cu") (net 1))
 (segment (start 133.2611 108.8136) (end 133.2611 106.2736) (width 0.4064) (layer "F.Cu") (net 1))
 (segment (start 140.8811 106.2736) (end 143.4211 106.2736) (width 0.4064) (layer "B.Cu") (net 1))
 (segment (start 151.0411 106.2736) (end 153.5811 106.2736) (width 0.4064) (layer "B.Cu") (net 1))
 (segment (start 148.5011 106.2736) (end 151.0411 106.2736) (width 0.4064) (layer "B.Cu") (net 1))
 (segment (start 128.1811 106.2736) (end 130.7211 106.2736) (width 0.4064) (layer "B.Cu") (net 1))
 (segment (start 163.7411 106.2736) (end 166.2811 106.2736) (width 0.4064) (layer "B.Cu") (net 1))
 (segment (start 156.1211 106.2736) (end 158.6611 106.2736) (width 0.4064) (layer "B.Cu") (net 1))
 (segment (start 130.7211 106.2736) (end 133.2611 106.2736) (width 0.4064) (layer "B.Cu") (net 1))
 (segment (start 135.8011 106.2736) (end 138.3411 106.2736) (width 0.4064) (layer "B.Cu") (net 1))
 (segment (start 133.3881 106.4006) (end 133.2611 106.2736) (width 0.4064) (layer "B.Cu") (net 1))
 (segment (start 135.8011 106.2736) (end 135.6741 106.4006) (width 0.4064) (layer "B.Cu") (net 1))
 (segment (start 135.6741 106.4006) (end 133.3881 106.4006) (width 0.4064) (layer "B.Cu") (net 1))
 (segment (start 158.6611 106.2736) (end 161.2011 106.2736) (width 0.4064) (layer "B.Cu") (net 1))
 (segment (start 145.9611 106.2736) (end 148.5011 106.2736) (width 0.4064) (layer "B.Cu") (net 1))
 (segment (start 138.3411 106.2736) (end 140.8811 106.2736) (width 0.4064) (layer "B.Cu") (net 1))
 (segment (start 163.7411 106.2736) (end 161.2011 106.2736) (width 0.4064) (layer "B.Cu") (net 1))
 (segment (start 166.2811 106.2736) (end 168.8211 106.2736) (width 0.4064) (layer "B.Cu") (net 1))
 (segment (start 143.4211 106.2736) (end 145.9611 106.2736) (width 0.4064) (layer "B.Cu") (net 1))
 (segment (start 153.5811 106.2736) (end 156.1211 106.2736) (width 0.4064) (layer "B.Cu") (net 1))
 (segment (start 134.5311 112.6236) (end 134.5311 115.1636) (width 0.4064) (layer "F.Cu") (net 17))
 (segment (start 129.4511 112.6236) (end 129.4511 115.1636) (width 0.4064) (layer "F.Cu") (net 15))
 (segment (start 139.6111 94.8436) (end 139.6111 97.3836) (width 0.4064) (layer "F.Cu") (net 28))
 (segment (start 142.1511 97.3836) (end 142.1511 94.8436) (width 0.4064) (layer "F.Cu") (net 27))
 (segment (start 144.6911 94.8436) (end 144.6911 97.3836) (width 0.4064) (layer "F.Cu") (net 26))
 (segment (start 135.4201 99.6696) (end 143.4211 99.6696) (width 0.4064) (layer "F.Cu") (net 26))
 (segment (start 134.5801 96.7486) (end 134.5801 98.8296) (width 0.4064) (layer "F.Cu") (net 26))
 (segment (start 143.4211 99.6696) (end 144.6911 98.3996) (width 0.4064) (layer "F.Cu") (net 26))
 (segment (start 134.5801 98.8296) (end 135.4201 99.6696) (width 0.4064) (layer "F.Cu") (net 26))
 (segment (start 144.6911 98.3996) (end 144.6911 97.3836) (width 0.4064) (layer "F.Cu") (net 26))
 (segment (start 165.0111 94.8436) (end 165.0111 97.3836) (width 0.4064) (layer "F.Cu") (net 25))
 (segment (start 154.8511 115.1636) (end 154.8511 112.6236) (width 0.4064) (layer "F.Cu") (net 18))
 (segment (start 157.3911 115.1636) (end 157.3911 112.6236) (width 0.4064) (layer "F.Cu") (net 19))
 (segment (start 159.9311 115.1636) (end 159.9311 112.6236) (width 0.4064) (layer "F.Cu") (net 20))
 (segment (start 162.4711 115.1636) (end 162.4711 112.6236) (width 0.4064) (layer "F.Cu") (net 21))
 (segment (start 165.0111 115.1636) (end 165.0111 112.6236) (width 0.4064) (layer "F.Cu") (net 22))
 (segment (start 167.5511 97.3836) (end 167.5511 94.8436) (width 0.4064) (layer "F.Cu") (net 24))
 (segment (start 139.6111 112.6236) (end 139.6111 115.1636) (width 0.4064) (layer "F.Cu") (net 2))
 (segment (start 134.1501 105.0036) (end 134.5311 105.3846) (width 0.254) (layer "F.Cu") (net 2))
 (segment (start 134.5311 107.5436) (end 139.6111 112.6236) (width 0.254) (layer "F.Cu") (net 2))
 (segment (start 128.1811 103.7336) (end 129.4511 105.0036) (width 0.254) (layer "F.Cu") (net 2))
 (segment (start 129.4511 105.0036) (end 134.1501 105.0036) (width 0.254) (layer "F.Cu") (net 2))
 (segment (start 134.5311 105.3846) (end 134.5311 107.5436) (width 0.254) (layer "F.Cu") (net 2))
 (segment (start 142.1511 115.1636) (end 142.1511 112.6236) (width 0.4064) (layer "F.Cu") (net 3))
 (segment (start 142.1511 109.267813) (end 142.1511 112.6236) (width 0.254) (layer "F.Cu") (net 3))
 (segment (start 133.7691 103.7336) (end 133.2611 103.7336) (width 0.254) (layer "F.Cu") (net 3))
 (segment (start 139.3571 105.0036) (end 135.0391 105.0036) (width 0.254) (layer "F.Cu") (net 3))
 (segment (start 135.0391 105.0036) (end 133.7691 103.7336) (width 0.254) (layer "F.Cu") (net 3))
 (segment (start 139.6619 105.3084) (end 139.6619 106.778613) (width 0.254) (layer "F.Cu") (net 3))
 (segment (start 139.6619 106.778613) (end 142.1511 109.267813) (width 0.254) (layer "F.Cu") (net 3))
 (segment (start 139.6619 105.3084) (end 139.3571 105.0036) (width 0.254) (layer "F.Cu") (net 3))
 (segment (start 143.926112 105.0544) (end 144.6911 105.819388) (width 0.254) (layer "F.Cu") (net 4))
 (segment (start 142.2019 105.0544) (end 143.926112 105.0544) (width 0.254) (layer "F.Cu") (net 4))
 (segment (start 144.6911 105.819388) (end 144.6911 112.6236) (width 0.254) (layer "F.Cu") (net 4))
 (segment (start 144.6911 112.6236) (end 144.6911 115.1636) (width 0.4064) (layer "F.Cu") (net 4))
 (segment (start 140.8811 103.7336) (end 142.2019 105.0544) (width 0.254) (layer "F.Cu") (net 4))
 (segment (start 147.2311 115.1636) (end 147.2311 112.6236) (width 0.4064) (layer "F.Cu") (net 5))
 (segment (start 145.9611 103.7336) (end 147.2311 105.0036) (width 0.254) (layer "F.Cu") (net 5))
 (segment (start 147.2311 105.0036) (end 147.2311 112.6236) (width 0.254) (layer "F.Cu") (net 5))
 (segment (start 149.7711 112.7506) (end 149.7711 112.6236) (width 0.4064) (layer "F.Cu") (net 6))
 (segment (start 149.7711 115.1636) (end 149.7711 112.7506) (width 0.4064) (layer "F.Cu") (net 6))
 (segment (start 148.5011 103.7336) (end 149.7711 105.0036) (width 0.254) (layer "F.Cu") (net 6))
 (segment (start 149.7711 105.0036) (end 149.7711 112.7506) (width 0.254) (layer "F.Cu") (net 6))
 (segment (start 151.0411 103.7336) (end 152.3111 105.0036) (width 0.254) (layer "F.Cu") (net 7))
 (segment (start 152.3111 115.1636) (end 152.3111 112.6236) (width 0.4064) (layer "F.Cu") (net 7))
 (segment (start 152.3111 105.0036) (end 152.3111 112.6236) (width 0.254) (layer "F.Cu") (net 7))
 (segment (start 152.3111 97.3836) (end 158.6611 103.7336) (width 0.254) (layer "F.Cu") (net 10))
 (segment (start 152.3111 94.8436) (end 152.3111 97.3836) (width 0.4064) (layer "F.Cu") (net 10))
 (segment (start 163.7411 103.7336) (end 165.0111 105.0036) (width 0.254) (layer "F.Cu") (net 12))
 (segment (start 157.3911 97.3836) (end 157.3911 94.8436) (width 0.4064) (layer "F.Cu") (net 12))
 (segment (start 165.0111 109.4096) (end 164.0561 110.4646) (width 0.254) (layer "F.Cu") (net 12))
 (segment (start 157.3911 97.3836) (end 163.7411 103.7336) (width 0.254) (layer "F.Cu") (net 12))
 (segment (start 165.0111 105.0036) (end 165.0111 109.4096) (width 0.254) (layer "F.Cu") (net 12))
 (segment (start 159.9311 97.3836) (end 166.2811 103.7336) (width 0.254) (layer "F.Cu") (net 13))
 (segment (start 159.9311 94.8436) (end 159.9311 97.3836) (width 0.4064) (layer "F.Cu") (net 13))
 (segment (start 162.4711 97.3836) (end 162.4711 94.8436) (width 0.4064) (layer "F.Cu") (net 14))
 (segment (start 168.8211 103.7336) (end 162.4711 97.3836) (width 0.254) (layer "F.Cu") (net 14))
 (segment (start 147.2311 97.3836) (end 153.5811 103.7336) (width 0.254) (layer "F.Cu") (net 8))
 (segment (start 147.2311 94.8436) (end 147.2311 97.3836) (width 0.4064) (layer "F.Cu") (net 8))
 (segment (start 149.7711 94.8436) (end 149.7711 97.3836) (width 0.4064) (layer "F.Cu") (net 9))
 (segment (start 149.7711 97.3836) (end 156.1211 103.7336) (width 0.254) (layer "F.Cu") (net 9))
 (segment (start 154.8511 97.3836) (end 161.2011 103.7336) (width 0.254) (layer "F.Cu") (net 11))
 (segment (start 154.8511 94.8436) (end 154.8511 97.3836) (width 0.4064) (layer "F.Cu") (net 11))
 (segment (start 162.1561 110.4646) (end 160.1851 110.4646) (width 0.254) (layer "F.Cu") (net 16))
 (segment (start 131.9911 115.1636) (end 131.9911 112.6236) (width 0.4064) (layer "F.Cu") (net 16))
 (via (at 160.1851 110.4646) (size 0.9064) (drill 0.5) (layers "F.Cu" "B.Cu") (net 16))
 (segment (start 131.9911 111.0996) (end 131.9911 112.6236) (width 0.254) (layer "B.Cu") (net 16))
 (segment (start 132.6261 110.4646) (end 131.9911 111.0996) (width 0.254) (layer "B.Cu") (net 16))
 (segment (start 160.1851 110.4646) (end 132.6261 110.4646) (width 0.254) (layer "B.Cu") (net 16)))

